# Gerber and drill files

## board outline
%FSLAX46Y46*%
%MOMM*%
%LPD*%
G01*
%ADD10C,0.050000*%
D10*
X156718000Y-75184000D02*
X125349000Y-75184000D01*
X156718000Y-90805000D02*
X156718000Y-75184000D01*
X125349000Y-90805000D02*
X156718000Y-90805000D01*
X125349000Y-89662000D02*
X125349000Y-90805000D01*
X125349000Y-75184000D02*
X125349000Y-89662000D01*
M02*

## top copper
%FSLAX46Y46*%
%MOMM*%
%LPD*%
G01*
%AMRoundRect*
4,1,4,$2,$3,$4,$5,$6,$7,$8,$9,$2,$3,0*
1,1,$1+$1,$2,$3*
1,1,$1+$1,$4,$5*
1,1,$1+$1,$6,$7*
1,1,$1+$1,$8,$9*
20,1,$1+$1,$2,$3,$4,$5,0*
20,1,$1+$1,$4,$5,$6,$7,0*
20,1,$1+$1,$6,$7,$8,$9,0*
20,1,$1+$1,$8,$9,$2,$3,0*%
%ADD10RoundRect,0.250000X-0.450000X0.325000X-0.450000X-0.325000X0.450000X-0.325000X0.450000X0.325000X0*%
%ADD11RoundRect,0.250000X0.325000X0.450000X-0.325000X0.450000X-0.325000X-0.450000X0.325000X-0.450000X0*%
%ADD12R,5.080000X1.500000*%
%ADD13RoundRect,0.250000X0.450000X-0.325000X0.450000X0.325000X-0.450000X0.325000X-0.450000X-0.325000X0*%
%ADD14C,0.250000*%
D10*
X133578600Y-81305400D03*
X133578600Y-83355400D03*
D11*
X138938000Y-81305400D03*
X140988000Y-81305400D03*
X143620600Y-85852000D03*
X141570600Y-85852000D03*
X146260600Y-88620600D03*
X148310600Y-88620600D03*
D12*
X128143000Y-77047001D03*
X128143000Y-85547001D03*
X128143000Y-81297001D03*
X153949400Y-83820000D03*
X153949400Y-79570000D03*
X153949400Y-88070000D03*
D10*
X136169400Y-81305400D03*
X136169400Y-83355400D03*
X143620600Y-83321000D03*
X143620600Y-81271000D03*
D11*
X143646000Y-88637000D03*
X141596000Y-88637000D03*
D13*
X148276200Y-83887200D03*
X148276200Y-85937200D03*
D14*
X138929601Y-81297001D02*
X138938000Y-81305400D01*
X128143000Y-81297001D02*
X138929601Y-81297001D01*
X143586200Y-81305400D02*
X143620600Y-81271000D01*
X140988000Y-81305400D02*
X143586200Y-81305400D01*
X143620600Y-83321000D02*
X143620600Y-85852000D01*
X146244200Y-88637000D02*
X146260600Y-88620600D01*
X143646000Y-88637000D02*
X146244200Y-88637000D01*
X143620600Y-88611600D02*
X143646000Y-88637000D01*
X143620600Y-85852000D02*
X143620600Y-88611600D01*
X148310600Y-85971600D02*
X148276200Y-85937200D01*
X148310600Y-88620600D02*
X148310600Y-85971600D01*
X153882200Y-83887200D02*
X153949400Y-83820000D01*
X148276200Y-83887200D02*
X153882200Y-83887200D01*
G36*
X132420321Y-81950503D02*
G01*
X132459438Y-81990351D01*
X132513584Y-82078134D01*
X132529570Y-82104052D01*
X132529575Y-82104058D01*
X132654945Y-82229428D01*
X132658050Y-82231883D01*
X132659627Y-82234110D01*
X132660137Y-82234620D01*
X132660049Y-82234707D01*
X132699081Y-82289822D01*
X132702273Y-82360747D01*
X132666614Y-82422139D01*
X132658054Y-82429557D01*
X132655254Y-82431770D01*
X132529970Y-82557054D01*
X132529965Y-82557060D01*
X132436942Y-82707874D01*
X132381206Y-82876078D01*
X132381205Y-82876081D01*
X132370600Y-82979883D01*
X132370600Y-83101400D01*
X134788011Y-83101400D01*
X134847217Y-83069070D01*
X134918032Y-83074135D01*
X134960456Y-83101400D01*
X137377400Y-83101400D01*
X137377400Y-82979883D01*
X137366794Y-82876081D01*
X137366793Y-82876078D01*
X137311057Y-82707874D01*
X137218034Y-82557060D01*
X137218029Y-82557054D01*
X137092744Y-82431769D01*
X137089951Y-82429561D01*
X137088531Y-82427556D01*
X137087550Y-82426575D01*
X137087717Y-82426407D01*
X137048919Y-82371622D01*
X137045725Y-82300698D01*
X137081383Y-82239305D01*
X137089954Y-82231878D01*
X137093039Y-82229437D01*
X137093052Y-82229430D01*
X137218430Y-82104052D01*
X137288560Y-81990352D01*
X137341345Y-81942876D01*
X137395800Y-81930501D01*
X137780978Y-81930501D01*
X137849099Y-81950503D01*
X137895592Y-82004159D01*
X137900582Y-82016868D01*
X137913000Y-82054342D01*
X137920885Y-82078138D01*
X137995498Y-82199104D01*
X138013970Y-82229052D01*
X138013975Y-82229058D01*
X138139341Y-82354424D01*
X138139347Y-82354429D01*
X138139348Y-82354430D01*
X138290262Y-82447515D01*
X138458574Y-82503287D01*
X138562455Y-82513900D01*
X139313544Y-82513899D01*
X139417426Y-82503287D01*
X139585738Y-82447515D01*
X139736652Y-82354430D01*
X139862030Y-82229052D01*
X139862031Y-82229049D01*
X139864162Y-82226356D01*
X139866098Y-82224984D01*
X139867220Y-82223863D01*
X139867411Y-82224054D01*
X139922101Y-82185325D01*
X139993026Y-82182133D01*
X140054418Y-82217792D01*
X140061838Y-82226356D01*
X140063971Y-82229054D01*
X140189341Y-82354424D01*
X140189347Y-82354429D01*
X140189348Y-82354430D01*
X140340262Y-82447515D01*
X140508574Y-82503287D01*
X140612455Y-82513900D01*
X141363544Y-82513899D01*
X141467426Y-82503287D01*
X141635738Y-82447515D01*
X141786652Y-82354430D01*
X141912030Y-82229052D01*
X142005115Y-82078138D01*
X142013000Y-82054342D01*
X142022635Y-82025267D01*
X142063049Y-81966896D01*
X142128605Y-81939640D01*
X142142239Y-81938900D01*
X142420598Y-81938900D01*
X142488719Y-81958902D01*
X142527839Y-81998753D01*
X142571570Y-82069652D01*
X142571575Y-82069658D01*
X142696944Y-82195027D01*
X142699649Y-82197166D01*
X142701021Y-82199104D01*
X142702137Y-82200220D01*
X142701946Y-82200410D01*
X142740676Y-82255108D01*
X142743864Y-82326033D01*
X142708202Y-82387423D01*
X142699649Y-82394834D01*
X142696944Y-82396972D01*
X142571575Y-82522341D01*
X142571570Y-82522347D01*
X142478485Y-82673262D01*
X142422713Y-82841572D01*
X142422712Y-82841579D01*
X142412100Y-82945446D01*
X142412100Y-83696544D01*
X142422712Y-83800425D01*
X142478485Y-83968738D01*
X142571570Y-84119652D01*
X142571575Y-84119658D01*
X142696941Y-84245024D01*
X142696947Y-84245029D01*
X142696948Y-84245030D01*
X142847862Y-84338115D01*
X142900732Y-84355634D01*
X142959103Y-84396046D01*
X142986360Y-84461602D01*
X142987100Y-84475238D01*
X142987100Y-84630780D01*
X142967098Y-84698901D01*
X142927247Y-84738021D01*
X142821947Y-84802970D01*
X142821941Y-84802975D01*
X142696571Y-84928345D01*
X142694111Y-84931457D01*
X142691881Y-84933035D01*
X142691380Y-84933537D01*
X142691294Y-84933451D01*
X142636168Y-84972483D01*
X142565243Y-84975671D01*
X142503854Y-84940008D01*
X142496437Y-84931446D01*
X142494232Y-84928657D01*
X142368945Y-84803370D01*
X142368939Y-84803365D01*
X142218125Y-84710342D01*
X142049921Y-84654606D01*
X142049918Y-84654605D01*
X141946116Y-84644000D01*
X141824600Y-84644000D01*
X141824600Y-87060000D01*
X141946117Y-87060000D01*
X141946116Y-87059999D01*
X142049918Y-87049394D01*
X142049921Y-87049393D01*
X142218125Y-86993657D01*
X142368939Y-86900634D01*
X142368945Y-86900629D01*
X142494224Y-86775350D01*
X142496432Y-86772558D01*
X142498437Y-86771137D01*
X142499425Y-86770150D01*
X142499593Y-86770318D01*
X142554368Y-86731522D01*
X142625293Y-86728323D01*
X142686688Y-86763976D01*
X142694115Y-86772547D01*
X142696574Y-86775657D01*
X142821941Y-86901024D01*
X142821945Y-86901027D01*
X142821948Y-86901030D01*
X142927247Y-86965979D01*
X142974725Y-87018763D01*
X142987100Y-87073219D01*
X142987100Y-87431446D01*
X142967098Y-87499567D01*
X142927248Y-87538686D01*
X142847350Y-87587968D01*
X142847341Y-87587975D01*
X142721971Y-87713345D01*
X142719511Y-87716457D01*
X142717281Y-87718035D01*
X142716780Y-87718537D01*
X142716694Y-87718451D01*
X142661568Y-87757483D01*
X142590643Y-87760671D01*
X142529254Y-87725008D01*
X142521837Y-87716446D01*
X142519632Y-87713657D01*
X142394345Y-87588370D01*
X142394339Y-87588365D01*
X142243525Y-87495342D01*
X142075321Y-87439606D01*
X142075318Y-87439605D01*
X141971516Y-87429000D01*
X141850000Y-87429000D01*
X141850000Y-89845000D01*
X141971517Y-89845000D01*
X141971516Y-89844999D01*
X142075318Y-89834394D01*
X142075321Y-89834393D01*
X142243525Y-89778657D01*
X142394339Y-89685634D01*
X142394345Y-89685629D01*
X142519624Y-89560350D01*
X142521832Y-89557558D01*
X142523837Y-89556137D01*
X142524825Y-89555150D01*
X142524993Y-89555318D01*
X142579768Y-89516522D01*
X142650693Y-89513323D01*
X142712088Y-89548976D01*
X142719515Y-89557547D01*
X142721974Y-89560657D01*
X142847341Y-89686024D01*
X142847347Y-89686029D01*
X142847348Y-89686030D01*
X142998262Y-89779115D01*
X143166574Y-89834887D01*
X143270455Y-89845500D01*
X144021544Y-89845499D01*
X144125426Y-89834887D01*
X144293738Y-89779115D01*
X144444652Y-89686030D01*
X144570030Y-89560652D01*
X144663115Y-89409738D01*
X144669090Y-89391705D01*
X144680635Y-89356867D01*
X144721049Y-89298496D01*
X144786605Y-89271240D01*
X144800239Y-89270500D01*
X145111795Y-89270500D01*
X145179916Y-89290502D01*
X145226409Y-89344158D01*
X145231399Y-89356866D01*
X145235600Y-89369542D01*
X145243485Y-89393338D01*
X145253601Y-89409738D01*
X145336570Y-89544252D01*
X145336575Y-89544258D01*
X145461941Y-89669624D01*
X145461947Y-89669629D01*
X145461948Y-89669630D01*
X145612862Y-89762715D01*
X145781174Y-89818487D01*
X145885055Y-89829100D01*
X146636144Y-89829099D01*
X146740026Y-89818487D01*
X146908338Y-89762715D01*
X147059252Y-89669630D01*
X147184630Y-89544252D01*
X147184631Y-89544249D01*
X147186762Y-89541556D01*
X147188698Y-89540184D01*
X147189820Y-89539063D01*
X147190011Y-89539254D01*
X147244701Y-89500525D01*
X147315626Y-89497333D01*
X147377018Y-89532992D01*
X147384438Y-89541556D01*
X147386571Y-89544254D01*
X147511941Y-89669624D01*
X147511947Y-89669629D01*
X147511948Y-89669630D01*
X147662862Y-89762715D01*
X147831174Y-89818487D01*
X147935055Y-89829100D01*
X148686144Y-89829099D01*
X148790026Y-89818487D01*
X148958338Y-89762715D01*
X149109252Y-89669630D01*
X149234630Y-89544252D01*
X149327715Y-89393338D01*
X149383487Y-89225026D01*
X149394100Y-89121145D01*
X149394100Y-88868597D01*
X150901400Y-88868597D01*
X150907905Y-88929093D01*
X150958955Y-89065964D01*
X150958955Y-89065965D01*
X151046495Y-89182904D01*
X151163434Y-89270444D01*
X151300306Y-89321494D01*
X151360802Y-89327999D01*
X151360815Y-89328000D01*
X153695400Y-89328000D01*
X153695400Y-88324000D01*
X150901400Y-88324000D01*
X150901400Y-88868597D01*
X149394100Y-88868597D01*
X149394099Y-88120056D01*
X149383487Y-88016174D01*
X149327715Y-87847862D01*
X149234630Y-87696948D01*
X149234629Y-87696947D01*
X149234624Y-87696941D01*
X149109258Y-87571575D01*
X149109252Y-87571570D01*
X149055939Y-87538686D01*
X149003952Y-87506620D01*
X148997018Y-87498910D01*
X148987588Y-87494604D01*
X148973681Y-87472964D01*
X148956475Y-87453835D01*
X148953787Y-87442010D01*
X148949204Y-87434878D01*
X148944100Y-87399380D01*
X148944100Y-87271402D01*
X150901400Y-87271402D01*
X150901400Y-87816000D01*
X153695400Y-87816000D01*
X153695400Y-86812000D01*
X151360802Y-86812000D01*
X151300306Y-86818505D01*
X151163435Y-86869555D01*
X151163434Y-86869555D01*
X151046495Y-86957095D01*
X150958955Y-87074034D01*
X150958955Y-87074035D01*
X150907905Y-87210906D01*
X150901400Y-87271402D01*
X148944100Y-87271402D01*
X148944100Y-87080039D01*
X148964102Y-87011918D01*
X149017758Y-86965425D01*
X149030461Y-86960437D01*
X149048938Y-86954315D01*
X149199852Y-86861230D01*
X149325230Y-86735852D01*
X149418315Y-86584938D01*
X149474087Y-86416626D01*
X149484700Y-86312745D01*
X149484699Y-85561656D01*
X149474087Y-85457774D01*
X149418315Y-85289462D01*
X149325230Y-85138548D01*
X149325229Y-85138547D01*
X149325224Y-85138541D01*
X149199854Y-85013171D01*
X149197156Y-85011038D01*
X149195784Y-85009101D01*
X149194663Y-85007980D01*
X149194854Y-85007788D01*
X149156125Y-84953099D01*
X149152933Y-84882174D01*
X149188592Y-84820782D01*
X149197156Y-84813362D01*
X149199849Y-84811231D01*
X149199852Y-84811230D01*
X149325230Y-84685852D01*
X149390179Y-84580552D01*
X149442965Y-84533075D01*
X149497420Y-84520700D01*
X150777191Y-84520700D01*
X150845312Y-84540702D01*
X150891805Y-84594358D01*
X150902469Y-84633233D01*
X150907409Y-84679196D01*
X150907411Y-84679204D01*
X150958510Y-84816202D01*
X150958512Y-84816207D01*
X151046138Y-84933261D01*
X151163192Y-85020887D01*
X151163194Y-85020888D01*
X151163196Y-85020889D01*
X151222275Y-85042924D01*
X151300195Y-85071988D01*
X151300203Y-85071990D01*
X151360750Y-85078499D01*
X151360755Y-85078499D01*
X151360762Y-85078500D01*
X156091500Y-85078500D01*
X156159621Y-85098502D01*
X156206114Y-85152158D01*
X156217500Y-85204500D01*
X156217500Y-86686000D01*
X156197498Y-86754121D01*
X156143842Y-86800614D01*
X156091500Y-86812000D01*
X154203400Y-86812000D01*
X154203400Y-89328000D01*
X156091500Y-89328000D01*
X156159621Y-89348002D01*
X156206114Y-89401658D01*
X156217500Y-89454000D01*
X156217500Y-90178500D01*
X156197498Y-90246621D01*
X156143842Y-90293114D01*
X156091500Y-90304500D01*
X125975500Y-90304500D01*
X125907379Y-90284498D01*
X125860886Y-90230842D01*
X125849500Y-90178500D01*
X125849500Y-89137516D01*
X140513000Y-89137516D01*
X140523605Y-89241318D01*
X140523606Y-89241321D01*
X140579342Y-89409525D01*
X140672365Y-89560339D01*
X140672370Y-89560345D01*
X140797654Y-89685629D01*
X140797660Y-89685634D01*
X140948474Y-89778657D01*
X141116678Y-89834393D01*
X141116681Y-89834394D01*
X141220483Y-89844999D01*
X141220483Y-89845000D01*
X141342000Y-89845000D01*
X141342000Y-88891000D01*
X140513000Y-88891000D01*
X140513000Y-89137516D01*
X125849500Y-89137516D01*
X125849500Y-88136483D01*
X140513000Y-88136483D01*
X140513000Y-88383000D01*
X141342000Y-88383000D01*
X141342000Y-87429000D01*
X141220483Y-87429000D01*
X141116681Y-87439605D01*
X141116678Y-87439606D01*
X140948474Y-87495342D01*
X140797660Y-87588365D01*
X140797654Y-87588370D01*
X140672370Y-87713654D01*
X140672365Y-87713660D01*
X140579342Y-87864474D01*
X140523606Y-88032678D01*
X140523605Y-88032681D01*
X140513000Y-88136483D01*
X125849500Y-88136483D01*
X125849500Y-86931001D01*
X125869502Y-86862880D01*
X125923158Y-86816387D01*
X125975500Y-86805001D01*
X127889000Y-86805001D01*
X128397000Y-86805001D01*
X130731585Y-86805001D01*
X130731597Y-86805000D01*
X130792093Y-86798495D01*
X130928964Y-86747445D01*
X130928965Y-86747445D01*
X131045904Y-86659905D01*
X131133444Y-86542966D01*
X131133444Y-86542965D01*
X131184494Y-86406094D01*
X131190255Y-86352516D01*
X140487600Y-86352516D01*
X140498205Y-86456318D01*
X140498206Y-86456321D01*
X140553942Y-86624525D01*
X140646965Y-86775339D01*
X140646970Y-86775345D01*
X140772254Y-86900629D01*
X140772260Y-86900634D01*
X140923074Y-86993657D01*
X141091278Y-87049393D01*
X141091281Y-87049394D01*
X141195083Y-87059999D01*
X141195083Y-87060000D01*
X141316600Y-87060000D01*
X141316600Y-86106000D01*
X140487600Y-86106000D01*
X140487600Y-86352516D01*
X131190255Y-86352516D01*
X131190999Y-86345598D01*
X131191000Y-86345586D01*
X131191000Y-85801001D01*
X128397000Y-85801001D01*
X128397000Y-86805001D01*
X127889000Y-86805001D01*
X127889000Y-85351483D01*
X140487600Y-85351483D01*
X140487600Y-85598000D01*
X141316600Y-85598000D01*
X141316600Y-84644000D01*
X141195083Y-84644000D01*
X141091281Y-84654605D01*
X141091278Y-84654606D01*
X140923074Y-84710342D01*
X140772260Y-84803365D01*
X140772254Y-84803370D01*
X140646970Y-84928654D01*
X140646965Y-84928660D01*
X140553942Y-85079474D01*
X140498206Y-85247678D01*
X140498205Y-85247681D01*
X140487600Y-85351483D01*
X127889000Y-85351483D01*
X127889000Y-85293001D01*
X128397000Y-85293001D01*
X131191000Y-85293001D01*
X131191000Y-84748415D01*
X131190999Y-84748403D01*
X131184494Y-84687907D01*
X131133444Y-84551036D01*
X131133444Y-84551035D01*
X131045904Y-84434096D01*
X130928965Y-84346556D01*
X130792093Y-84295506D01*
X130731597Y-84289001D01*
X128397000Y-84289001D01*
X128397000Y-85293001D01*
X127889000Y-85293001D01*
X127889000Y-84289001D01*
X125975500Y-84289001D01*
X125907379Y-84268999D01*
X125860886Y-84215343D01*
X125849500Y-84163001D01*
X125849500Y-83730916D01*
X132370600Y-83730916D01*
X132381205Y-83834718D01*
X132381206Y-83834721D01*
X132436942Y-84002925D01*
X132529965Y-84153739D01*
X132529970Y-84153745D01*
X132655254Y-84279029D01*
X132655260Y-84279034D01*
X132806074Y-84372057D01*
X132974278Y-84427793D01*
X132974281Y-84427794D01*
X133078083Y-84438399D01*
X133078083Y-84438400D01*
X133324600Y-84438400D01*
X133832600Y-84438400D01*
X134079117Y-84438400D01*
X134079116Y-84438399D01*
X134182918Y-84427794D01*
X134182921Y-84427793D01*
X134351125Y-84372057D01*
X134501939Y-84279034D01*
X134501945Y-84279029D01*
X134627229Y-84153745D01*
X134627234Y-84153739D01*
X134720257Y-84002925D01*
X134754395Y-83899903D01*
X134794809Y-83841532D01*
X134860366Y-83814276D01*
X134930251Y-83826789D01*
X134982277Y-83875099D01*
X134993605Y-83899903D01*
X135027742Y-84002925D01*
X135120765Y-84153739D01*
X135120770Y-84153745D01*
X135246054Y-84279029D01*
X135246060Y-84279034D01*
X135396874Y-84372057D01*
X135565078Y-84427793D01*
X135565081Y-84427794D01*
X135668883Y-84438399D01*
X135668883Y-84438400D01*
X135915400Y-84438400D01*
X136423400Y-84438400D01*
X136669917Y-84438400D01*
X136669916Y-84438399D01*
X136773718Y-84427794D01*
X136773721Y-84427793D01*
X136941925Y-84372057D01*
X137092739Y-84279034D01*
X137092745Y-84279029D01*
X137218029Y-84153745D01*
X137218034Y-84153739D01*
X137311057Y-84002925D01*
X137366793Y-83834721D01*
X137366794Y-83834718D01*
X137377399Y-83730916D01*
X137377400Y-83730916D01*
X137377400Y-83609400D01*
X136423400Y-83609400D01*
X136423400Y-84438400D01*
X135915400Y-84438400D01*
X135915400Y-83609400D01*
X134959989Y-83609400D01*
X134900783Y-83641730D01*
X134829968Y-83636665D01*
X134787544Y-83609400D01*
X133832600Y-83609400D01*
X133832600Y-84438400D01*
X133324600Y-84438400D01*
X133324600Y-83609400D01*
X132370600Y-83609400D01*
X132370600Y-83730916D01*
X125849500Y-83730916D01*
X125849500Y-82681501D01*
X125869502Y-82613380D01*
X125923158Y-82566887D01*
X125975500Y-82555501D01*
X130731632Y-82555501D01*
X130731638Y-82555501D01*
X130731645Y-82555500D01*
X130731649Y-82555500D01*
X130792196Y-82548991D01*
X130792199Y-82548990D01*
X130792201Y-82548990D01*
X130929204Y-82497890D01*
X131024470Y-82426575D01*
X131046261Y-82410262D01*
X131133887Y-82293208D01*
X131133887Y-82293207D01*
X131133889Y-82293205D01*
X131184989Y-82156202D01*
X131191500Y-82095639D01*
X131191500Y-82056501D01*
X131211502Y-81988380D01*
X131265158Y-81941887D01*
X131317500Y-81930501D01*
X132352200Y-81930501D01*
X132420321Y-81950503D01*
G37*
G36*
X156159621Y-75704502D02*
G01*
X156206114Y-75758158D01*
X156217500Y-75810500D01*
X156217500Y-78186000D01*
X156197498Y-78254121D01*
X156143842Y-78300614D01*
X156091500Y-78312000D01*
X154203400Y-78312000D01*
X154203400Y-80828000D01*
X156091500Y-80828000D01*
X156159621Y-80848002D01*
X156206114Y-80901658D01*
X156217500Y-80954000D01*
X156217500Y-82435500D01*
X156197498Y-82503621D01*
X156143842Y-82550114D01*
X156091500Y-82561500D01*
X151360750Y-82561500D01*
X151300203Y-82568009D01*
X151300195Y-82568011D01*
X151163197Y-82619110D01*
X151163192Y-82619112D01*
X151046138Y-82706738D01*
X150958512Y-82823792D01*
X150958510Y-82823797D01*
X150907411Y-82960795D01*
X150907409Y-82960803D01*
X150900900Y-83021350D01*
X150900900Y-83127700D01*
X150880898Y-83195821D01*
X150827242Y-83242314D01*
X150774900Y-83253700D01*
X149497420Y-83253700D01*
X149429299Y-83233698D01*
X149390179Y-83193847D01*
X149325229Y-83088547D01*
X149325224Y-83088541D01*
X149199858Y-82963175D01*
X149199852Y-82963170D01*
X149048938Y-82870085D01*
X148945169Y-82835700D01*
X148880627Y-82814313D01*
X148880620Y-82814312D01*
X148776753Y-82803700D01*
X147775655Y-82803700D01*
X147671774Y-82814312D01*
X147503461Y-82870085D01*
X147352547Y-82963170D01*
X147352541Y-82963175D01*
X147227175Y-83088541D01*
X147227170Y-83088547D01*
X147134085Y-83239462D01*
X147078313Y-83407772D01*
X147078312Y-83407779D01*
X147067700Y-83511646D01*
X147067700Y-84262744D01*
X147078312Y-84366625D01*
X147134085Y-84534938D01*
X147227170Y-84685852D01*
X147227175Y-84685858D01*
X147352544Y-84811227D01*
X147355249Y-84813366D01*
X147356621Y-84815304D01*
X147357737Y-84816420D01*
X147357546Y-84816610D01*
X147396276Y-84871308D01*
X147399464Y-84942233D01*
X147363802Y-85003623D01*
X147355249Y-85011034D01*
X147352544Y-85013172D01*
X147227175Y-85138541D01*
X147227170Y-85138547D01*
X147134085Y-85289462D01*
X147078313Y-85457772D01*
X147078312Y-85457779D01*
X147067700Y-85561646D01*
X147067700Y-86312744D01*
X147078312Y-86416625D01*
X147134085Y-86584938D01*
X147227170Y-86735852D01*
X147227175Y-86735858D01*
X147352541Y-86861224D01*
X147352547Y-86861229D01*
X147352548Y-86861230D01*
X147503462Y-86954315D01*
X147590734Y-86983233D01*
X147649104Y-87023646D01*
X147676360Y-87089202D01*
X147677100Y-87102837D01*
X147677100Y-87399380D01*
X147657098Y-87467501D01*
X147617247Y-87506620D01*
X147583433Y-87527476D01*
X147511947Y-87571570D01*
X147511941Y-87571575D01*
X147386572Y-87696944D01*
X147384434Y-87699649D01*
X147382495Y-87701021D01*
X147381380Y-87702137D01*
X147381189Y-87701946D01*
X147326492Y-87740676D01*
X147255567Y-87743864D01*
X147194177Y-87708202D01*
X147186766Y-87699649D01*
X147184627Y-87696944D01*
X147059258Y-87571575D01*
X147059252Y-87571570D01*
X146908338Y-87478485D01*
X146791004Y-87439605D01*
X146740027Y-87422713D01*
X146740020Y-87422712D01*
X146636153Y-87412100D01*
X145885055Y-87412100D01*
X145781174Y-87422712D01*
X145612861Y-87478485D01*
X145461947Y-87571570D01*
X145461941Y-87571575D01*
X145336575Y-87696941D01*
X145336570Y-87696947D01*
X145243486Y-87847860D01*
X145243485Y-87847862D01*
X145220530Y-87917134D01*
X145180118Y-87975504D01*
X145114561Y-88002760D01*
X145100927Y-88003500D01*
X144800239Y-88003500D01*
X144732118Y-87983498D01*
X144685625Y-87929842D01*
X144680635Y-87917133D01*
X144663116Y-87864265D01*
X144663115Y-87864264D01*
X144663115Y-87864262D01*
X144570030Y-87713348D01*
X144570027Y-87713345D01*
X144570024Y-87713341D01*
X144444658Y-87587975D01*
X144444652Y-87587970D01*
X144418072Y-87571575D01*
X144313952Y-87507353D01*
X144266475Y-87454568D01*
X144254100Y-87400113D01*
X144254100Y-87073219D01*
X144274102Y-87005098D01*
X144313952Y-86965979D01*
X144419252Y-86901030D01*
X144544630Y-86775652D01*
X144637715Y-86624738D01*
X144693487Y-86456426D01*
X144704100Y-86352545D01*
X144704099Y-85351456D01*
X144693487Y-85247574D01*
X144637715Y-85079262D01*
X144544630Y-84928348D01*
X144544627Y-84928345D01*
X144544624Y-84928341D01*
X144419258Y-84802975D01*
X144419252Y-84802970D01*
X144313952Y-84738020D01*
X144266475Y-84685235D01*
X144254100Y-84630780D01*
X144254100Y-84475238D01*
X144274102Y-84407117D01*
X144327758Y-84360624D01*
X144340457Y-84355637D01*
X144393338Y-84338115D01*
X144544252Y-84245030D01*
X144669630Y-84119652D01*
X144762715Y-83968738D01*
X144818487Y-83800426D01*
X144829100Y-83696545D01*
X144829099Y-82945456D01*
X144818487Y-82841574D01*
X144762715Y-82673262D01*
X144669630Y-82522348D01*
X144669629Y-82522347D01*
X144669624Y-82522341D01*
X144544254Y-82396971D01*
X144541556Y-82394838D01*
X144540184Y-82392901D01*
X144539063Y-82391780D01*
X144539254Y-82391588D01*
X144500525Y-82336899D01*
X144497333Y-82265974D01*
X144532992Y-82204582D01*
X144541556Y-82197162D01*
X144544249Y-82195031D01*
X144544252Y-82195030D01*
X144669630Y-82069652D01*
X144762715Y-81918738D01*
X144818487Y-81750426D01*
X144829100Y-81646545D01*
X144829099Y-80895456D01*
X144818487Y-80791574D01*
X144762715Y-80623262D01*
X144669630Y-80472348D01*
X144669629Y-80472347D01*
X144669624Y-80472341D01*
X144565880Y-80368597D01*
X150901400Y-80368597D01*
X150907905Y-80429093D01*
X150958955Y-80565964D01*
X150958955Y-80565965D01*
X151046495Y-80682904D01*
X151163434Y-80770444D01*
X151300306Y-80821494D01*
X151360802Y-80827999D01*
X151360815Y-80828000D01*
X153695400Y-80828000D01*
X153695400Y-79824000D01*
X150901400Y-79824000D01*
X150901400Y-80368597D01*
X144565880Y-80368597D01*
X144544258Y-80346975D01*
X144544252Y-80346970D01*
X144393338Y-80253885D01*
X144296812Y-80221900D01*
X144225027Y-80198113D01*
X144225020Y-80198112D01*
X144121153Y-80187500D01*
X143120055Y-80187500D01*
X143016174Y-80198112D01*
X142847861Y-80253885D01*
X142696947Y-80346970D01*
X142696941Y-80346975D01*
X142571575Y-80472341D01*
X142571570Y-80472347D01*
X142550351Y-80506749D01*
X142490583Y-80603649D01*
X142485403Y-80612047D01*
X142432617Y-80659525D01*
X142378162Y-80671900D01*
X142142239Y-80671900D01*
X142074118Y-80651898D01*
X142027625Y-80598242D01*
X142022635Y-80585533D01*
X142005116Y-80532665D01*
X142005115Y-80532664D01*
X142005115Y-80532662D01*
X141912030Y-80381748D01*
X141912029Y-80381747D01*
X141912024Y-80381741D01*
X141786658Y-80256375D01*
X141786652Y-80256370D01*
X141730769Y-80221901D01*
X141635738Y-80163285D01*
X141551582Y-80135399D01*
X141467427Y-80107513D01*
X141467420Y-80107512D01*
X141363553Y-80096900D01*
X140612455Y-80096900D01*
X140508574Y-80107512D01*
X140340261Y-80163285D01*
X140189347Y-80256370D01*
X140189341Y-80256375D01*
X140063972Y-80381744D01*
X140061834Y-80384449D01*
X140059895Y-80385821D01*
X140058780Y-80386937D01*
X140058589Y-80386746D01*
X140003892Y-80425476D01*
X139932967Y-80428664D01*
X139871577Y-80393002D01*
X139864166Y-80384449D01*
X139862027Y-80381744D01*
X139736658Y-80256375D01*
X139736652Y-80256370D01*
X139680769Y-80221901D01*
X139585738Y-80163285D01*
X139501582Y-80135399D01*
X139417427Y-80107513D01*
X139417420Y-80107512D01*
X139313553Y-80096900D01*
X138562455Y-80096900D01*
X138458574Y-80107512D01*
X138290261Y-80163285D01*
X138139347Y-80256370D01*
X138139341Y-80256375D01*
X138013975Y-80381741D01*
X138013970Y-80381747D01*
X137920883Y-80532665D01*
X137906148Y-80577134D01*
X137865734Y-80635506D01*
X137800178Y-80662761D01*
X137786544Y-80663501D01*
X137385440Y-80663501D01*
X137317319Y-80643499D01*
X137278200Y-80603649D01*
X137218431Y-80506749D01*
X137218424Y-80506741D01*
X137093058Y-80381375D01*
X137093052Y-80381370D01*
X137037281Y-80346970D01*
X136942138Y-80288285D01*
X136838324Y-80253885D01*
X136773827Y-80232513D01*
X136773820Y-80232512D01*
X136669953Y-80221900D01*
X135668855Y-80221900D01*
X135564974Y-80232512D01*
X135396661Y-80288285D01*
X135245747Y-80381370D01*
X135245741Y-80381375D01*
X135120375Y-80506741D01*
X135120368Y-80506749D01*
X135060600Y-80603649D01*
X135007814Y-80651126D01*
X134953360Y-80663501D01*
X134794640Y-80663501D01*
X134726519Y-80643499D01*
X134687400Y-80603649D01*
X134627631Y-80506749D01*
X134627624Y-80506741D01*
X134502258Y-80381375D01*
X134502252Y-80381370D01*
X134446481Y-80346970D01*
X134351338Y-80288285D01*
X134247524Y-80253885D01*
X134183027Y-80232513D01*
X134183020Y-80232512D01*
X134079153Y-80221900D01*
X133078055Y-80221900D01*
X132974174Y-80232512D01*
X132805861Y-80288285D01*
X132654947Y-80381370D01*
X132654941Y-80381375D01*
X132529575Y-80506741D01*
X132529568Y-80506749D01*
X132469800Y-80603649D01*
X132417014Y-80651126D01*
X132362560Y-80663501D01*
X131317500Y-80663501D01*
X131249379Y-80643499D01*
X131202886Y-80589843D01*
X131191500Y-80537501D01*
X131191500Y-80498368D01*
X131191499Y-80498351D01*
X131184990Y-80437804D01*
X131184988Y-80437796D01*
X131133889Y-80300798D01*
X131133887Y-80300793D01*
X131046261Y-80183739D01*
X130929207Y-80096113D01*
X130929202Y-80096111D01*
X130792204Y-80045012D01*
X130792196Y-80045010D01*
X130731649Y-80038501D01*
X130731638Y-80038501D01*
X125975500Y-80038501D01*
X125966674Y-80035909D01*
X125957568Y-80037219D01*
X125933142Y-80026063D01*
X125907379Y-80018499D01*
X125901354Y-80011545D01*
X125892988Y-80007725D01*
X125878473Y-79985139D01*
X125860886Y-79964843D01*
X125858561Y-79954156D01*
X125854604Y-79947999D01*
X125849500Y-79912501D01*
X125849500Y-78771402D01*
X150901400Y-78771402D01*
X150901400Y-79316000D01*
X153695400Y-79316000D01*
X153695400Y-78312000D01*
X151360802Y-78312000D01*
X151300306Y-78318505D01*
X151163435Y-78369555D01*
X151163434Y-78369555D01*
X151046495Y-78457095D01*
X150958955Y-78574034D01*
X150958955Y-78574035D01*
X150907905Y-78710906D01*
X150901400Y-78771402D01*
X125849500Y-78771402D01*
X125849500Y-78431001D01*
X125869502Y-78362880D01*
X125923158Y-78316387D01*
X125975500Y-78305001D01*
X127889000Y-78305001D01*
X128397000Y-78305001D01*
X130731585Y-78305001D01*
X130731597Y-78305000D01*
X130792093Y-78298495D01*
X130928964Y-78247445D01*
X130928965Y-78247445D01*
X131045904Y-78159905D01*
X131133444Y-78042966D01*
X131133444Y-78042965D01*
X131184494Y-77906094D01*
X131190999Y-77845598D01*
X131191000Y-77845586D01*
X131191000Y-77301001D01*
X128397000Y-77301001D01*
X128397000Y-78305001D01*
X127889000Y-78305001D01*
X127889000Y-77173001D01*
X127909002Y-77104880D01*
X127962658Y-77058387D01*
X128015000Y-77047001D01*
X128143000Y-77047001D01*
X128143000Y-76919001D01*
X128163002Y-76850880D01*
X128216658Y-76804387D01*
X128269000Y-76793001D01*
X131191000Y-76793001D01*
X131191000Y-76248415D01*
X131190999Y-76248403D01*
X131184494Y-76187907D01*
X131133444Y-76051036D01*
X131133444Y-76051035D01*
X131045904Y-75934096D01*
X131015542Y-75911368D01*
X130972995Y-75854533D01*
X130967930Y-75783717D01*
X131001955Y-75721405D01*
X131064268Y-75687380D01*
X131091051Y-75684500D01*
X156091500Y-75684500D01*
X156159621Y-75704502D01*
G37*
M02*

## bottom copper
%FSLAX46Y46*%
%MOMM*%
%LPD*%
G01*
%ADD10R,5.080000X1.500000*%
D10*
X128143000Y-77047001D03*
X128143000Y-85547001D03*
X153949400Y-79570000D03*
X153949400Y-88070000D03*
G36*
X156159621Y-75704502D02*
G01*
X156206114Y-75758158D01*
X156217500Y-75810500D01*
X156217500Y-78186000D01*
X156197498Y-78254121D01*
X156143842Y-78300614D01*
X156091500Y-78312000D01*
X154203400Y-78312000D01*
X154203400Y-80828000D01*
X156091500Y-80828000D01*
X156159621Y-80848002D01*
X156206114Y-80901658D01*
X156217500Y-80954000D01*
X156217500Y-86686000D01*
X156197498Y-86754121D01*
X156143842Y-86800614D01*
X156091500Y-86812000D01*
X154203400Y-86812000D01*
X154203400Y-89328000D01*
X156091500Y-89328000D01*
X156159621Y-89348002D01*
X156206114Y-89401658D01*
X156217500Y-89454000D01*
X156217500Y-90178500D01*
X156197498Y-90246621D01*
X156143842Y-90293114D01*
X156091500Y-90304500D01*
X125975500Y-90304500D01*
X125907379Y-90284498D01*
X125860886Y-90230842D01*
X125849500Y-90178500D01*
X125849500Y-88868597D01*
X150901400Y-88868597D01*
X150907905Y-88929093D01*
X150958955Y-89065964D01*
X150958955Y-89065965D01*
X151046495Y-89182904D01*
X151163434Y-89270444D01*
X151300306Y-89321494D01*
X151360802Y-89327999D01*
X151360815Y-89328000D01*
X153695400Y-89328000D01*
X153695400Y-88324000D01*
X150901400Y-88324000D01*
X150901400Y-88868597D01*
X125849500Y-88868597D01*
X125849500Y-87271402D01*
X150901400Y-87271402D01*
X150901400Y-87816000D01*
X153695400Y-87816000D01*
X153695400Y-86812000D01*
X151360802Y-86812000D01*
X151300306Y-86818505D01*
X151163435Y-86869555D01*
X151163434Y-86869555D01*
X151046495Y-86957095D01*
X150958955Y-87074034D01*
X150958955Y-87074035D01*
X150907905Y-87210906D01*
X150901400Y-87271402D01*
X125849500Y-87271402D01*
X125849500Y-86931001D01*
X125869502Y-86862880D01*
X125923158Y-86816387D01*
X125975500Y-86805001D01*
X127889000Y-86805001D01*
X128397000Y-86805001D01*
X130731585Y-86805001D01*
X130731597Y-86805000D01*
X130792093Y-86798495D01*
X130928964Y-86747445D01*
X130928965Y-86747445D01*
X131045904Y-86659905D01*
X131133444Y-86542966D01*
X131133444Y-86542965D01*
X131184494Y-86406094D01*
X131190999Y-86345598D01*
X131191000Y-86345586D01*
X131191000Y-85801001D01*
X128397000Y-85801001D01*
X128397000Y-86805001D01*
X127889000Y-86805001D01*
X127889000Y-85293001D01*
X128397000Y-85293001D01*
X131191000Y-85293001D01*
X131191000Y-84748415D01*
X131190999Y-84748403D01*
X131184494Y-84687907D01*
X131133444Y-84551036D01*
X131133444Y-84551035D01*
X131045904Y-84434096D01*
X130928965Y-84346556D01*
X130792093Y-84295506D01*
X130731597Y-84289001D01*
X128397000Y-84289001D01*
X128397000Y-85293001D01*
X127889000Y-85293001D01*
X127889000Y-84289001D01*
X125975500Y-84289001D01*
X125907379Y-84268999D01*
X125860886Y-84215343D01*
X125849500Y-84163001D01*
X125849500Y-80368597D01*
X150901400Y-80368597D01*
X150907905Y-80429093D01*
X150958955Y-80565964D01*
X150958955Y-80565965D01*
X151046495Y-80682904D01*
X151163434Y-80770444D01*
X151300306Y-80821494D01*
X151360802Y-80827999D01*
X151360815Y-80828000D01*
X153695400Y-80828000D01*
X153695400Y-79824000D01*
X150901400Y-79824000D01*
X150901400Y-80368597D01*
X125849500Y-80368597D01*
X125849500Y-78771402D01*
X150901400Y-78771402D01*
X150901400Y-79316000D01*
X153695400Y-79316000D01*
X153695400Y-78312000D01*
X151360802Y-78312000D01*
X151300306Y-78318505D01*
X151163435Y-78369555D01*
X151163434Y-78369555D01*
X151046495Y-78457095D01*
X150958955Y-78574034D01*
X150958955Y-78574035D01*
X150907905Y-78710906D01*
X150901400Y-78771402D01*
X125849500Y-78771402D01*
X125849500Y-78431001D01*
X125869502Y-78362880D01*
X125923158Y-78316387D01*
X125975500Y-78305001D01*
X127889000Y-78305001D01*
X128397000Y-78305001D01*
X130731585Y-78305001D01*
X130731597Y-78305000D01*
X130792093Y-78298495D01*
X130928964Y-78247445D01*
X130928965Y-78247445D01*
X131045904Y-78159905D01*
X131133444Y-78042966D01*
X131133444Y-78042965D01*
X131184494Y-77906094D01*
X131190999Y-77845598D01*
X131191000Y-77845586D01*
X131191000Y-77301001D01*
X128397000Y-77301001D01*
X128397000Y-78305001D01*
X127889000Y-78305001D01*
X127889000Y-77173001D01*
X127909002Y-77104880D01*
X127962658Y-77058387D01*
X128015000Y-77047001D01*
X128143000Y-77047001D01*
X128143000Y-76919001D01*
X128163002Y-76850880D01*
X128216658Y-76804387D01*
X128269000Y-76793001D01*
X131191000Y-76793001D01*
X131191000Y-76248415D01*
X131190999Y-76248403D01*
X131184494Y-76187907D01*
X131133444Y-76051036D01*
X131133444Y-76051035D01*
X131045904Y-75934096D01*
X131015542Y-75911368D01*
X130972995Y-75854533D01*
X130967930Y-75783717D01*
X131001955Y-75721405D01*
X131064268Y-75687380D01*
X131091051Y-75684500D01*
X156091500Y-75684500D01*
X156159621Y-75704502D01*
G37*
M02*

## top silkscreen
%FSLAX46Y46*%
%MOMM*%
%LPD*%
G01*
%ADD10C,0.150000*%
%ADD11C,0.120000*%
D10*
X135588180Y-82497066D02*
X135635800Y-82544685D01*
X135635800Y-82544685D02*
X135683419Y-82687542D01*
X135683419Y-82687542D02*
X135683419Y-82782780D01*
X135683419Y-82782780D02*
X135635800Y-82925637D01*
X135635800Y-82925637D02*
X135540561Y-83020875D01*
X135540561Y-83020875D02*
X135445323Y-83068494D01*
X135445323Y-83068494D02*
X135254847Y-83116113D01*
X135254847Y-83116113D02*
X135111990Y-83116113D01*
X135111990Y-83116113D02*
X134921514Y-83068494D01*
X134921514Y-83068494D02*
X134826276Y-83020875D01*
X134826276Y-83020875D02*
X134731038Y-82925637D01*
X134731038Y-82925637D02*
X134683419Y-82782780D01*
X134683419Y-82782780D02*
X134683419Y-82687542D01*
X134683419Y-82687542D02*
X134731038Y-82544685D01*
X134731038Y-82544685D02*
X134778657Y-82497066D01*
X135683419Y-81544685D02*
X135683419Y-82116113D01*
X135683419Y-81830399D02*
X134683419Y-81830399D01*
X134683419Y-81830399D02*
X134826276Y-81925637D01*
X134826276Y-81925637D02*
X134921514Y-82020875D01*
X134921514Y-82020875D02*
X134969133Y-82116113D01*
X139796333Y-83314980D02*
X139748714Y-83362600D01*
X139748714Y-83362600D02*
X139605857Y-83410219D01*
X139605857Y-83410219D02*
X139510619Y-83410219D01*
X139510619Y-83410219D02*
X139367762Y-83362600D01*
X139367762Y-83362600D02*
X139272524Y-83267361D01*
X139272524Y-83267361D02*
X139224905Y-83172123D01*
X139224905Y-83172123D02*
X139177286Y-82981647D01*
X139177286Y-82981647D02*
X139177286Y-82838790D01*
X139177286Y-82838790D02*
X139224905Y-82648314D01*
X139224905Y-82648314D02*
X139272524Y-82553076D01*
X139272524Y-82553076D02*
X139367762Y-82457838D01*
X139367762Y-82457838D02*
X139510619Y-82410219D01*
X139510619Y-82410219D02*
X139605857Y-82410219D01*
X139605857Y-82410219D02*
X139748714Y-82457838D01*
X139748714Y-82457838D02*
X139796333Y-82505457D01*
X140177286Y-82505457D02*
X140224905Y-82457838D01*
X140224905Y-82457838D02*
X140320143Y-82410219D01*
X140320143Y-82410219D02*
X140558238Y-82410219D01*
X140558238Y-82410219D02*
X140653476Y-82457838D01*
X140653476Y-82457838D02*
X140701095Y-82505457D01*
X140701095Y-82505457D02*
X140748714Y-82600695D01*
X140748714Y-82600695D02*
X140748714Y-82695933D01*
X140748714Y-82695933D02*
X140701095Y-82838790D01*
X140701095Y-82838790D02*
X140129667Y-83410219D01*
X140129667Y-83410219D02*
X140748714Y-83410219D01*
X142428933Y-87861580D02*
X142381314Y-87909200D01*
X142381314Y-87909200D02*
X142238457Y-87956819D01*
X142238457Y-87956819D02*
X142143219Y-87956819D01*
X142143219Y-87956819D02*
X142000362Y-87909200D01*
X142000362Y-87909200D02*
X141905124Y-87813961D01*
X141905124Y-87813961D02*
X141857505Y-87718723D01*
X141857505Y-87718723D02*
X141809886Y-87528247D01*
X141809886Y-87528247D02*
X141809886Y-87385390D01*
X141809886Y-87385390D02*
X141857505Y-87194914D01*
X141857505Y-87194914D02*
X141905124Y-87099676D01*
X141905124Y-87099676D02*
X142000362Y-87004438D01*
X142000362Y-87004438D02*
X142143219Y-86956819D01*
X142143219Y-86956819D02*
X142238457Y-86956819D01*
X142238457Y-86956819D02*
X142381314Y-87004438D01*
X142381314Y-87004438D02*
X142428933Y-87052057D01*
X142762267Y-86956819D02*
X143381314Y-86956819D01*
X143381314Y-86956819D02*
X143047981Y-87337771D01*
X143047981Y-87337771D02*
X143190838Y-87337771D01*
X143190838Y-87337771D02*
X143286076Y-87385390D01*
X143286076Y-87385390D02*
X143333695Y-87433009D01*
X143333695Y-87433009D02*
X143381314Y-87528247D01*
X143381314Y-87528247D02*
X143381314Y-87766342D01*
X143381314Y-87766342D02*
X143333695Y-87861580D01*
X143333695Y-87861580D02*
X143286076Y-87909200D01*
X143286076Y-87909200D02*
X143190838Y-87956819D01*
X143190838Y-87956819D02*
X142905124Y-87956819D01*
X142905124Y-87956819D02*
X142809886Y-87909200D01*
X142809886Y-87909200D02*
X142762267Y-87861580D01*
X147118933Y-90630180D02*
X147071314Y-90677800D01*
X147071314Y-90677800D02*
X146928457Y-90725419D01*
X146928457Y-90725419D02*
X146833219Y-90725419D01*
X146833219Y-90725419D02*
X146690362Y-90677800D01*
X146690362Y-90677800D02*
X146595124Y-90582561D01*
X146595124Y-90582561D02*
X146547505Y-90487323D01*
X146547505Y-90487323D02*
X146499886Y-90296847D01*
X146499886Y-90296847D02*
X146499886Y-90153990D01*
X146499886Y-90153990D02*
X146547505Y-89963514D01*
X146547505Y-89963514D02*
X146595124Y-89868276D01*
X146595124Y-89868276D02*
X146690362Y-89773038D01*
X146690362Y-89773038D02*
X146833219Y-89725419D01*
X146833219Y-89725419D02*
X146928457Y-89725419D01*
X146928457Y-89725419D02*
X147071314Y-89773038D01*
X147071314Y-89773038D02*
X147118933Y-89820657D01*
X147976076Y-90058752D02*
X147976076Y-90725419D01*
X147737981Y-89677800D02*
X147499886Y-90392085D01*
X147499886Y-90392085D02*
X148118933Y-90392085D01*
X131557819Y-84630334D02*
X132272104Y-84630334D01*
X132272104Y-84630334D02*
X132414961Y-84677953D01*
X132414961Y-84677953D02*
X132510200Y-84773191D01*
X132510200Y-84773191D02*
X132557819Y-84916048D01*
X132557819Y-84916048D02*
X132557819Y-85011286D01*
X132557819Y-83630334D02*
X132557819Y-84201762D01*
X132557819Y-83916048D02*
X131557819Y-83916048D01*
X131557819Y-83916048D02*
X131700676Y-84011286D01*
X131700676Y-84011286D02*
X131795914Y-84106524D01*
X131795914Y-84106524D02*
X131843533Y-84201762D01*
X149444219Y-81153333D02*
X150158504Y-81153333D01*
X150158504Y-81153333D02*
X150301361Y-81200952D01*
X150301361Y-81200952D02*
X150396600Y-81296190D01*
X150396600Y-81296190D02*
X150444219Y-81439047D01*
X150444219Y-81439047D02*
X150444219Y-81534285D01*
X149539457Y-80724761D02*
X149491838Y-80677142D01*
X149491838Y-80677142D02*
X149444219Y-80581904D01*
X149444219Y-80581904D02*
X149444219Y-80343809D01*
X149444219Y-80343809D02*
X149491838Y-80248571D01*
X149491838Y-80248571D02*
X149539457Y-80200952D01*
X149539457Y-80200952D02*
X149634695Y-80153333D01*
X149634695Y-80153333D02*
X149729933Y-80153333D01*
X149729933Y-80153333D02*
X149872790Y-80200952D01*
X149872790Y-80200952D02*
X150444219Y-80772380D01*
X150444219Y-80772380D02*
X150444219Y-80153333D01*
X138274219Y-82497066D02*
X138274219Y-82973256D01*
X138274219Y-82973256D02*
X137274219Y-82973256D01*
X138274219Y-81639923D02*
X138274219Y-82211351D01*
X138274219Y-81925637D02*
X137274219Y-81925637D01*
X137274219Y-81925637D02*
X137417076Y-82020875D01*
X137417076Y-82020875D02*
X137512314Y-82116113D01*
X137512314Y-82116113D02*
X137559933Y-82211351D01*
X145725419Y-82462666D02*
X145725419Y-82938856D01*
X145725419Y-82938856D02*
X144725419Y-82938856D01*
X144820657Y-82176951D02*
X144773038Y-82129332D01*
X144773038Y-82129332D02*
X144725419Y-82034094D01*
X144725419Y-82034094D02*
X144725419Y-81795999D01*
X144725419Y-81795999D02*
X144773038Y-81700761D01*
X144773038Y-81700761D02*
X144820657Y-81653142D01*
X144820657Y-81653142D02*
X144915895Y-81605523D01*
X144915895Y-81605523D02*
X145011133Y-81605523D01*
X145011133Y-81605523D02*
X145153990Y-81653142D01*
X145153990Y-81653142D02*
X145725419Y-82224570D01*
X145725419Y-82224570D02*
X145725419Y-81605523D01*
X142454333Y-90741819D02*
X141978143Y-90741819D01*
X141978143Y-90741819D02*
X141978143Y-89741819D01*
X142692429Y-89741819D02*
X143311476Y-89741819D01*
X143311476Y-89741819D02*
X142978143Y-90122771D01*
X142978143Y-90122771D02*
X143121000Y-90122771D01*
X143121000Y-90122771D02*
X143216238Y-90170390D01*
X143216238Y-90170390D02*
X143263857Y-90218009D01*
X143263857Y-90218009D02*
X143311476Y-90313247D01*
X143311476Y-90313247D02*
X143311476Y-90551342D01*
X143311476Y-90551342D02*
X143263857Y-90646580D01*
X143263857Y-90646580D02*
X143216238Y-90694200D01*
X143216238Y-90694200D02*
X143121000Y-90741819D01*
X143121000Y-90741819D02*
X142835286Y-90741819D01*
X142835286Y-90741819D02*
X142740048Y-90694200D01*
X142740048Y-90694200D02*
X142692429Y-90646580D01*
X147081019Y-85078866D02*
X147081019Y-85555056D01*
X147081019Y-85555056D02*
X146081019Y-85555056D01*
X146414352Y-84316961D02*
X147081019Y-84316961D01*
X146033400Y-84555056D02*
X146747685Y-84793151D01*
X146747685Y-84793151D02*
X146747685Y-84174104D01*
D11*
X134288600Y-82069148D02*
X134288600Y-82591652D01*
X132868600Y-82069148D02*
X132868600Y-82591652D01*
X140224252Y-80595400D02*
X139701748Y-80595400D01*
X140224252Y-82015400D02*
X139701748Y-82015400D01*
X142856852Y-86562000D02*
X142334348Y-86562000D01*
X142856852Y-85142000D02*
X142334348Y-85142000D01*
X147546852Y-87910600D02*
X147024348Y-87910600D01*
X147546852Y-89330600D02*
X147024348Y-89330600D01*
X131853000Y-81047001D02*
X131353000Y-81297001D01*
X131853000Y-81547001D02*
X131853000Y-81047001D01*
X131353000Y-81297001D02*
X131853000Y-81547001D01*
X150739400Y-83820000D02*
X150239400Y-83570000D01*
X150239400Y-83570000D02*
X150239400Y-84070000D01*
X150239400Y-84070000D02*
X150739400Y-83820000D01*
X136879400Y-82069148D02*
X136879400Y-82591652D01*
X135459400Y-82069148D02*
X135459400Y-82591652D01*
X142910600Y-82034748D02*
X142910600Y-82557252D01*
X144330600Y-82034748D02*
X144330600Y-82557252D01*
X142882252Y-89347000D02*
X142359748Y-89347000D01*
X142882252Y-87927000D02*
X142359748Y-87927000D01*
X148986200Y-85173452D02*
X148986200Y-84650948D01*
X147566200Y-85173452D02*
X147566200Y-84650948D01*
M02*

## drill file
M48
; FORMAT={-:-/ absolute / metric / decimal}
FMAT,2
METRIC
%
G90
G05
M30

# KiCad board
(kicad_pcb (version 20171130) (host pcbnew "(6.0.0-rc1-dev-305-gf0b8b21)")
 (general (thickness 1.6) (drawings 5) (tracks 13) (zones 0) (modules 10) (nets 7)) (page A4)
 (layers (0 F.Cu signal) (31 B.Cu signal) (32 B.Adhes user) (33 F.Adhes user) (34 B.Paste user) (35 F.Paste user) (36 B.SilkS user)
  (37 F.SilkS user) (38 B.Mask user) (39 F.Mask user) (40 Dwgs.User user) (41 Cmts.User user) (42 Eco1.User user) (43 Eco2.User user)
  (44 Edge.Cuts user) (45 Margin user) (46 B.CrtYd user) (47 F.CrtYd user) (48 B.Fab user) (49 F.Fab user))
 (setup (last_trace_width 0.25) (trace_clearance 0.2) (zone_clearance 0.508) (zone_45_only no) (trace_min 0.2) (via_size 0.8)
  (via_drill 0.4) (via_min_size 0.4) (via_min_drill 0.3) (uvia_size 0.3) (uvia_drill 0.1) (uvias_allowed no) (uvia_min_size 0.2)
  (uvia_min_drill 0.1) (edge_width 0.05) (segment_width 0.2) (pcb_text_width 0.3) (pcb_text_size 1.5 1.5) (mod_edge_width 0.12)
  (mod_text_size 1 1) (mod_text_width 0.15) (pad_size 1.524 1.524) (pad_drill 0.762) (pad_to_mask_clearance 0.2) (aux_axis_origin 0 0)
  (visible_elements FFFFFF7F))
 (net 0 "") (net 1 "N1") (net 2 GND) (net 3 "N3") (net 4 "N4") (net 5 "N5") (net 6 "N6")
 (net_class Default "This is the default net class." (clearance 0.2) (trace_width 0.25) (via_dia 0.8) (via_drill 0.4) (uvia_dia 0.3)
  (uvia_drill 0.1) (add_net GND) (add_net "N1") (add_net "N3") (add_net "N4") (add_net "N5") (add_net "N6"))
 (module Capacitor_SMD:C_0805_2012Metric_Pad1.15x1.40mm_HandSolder (layer F.Cu) (at 133.5786 82.3304 270)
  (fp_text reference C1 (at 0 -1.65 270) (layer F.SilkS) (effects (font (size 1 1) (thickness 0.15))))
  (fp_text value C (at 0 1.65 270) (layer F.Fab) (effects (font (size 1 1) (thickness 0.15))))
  (fp_line (start -0.261252 -0.71) (end 0.261252 -0.71) (layer F.SilkS) (width 0.12))
  (fp_line (start -0.261252 0.71) (end 0.261252 0.71) (layer F.SilkS) (width 0.12))
  (pad 1 smd roundrect (at -1.025 0 270) (size 1.15 1.4) (layers F.Cu F.Paste F.Mask) (roundrect_rratio 0.217391) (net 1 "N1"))
  (pad 2 smd roundrect (at 1.025 0 270) (size 1.15 1.4) (layers F.Cu F.Paste F.Mask) (roundrect_rratio 0.217391) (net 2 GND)))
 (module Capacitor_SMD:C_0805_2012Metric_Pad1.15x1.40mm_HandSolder (layer F.Cu) (at 139.963 81.3054 180)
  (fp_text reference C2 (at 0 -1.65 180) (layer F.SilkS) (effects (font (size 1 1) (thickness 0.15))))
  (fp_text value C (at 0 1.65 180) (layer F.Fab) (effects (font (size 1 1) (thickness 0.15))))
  (fp_line (start -0.261252 0.71) (end 0.261252 0.71) (layer F.SilkS) (width 0.12))
  (fp_line (start -0.261252 -0.71) (end 0.261252 -0.71) (layer F.SilkS) (width 0.12))
  (pad 2 smd roundrect (at 1.025 0 180) (size 1.15 1.4) (layers F.Cu F.Paste F.Mask) (roundrect_rratio 0.217391) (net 1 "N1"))
  (pad 1 smd roundrect (at -1.025 0 180) (size 1.15 1.4) (layers F.Cu F.Paste F.Mask) (roundrect_rratio 0.217391) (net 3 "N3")))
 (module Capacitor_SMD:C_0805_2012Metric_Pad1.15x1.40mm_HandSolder (layer F.Cu) (at 142.5956 85.852 180)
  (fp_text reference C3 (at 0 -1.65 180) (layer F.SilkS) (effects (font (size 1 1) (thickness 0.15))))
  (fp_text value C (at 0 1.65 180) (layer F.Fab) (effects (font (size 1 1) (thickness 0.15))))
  (fp_line (start -0.261252 -0.71) (end 0.261252 -0.71) (layer F.SilkS) (width 0.12))
  (fp_line (start -0.261252 0.71) (end 0.261252 0.71) (layer F.SilkS) (width 0.12))
  (pad 1 smd roundrect (at -1.025 0 180) (size 1.15 1.4) (layers F.Cu F.Paste F.Mask) (roundrect_rratio 0.217391) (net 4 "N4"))
  (pad 2 smd roundrect (at 1.025 0 180) (size 1.15 1.4) (layers F.Cu F.Paste F.Mask) (roundrect_rratio 0.217391) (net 2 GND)))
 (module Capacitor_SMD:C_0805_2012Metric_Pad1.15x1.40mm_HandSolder (layer F.Cu) (at 147.2856 88.6206 180)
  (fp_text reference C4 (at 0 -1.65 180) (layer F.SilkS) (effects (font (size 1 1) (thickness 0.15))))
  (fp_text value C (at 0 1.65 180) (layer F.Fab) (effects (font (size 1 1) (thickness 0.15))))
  (fp_line (start -0.261252 0.71) (end 0.261252 0.71) (layer F.SilkS) (width 0.12))
  (fp_line (start -0.261252 -0.71) (end 0.261252 -0.71) (layer F.SilkS) (width 0.12))
  (pad 2 smd roundrect (at 1.025 0 180) (size 1.15 1.4) (layers F.Cu F.Paste F.Mask) (roundrect_rratio 0.217391) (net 4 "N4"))
  (pad 1 smd roundrect (at -1.025 0 180) (size 1.15 1.4) (layers F.Cu F.Paste F.Mask) (roundrect_rratio 0.217391) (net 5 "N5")))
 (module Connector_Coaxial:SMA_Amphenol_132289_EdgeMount (layer F.Cu) (at 128.143 81.297001 180)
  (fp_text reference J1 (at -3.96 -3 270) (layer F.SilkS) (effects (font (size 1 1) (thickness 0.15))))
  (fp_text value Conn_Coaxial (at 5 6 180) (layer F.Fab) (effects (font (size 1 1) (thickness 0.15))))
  (fp_line (start -3.71 0.25) (end -3.21 0) (layer F.SilkS) (width 0.12))
  (fp_line (start -3.71 -0.25) (end -3.71 0.25) (layer F.SilkS) (width 0.12))
  (fp_line (start -3.21 0) (end -3.71 -0.25) (layer F.SilkS) (width 0.12))
  (pad 2 smd rect (at 0 4.25 270) (size 1.5 5.08) (layers B.Cu B.Paste B.Mask) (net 2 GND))
  (pad 2 smd rect (at 0 -4.25 270) (size 1.5 5.08) (layers B.Cu B.Paste B.Mask) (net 2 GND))
  (pad 2 smd rect (at 0 4.25 270) (size 1.5 5.08) (layers F.Cu F.Paste F.Mask) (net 2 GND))
  (pad 2 smd rect (at 0 -4.25 270) (size 1.5 5.08) (layers F.Cu F.Paste F.Mask) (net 2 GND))
  (pad 1 smd rect (at 0 0 270) (size 1.5 5.08) (layers F.Cu F.Paste F.Mask) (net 1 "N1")))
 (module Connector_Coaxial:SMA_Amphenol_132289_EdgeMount (layer F.Cu) (at 153.9494 83.82)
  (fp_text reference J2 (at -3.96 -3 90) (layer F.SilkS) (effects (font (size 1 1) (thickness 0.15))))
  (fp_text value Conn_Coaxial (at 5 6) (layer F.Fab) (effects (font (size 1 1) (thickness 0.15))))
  (fp_line (start -3.21 0) (end -3.71 -0.25) (layer F.SilkS) (width 0.12))
  (fp_line (start -3.71 -0.25) (end -3.71 0.25) (layer F.SilkS) (width 0.12))
  (fp_line (start -3.71 0.25) (end -3.21 0) (layer F.SilkS) (width 0.12))
  (pad 1 smd rect (at 0 0 90) (size 1.5 5.08) (layers F.Cu F.Paste F.Mask) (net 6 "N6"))
  (pad 2 smd rect (at 0 -4.25 90) (size 1.5 5.08) (layers F.Cu F.Paste F.Mask) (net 2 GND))
  (pad 2 smd rect (at 0 4.25 90) (size 1.5 5.08) (layers F.Cu F.Paste F.Mask) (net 2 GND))
  (pad 2 smd rect (at 0 -4.25 90) (size 1.5 5.08) (layers B.Cu B.Paste B.Mask) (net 2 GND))
  (pad 2 smd rect (at 0 4.25 90) (size 1.5 5.08) (layers B.Cu B.Paste B.Mask) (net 2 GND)))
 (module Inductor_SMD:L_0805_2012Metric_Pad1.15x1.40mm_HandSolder (layer F.Cu) (at 136.1694 82.3304 270)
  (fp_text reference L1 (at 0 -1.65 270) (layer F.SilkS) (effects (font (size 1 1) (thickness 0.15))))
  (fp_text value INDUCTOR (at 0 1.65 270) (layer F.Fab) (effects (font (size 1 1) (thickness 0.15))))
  (fp_line (start -0.261252 -0.71) (end 0.261252 -0.71) (layer F.SilkS) (width 0.12))
  (fp_line (start -0.261252 0.71) (end 0.261252 0.71) (layer F.SilkS) (width 0.12))
  (pad 1 smd roundrect (at -1.025 0 270) (size 1.15 1.4) (layers F.Cu F.Paste F.Mask) (roundrect_rratio 0.217391) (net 1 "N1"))
  (pad 2 smd roundrect (at 1.025 0 270) (size 1.15 1.4) (layers F.Cu F.Paste F.Mask) (roundrect_rratio 0.217391) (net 2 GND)))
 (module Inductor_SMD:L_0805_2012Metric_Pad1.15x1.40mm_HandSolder (layer F.Cu) (at 143.6206 82.296 270)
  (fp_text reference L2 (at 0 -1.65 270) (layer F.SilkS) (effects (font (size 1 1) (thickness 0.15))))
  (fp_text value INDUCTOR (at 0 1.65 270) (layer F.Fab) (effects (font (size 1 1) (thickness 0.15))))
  (fp_line (start -0.261252 0.71) (end 0.261252 0.71) (layer F.SilkS) (width 0.12))
  (fp_line (start -0.261252 -0.71) (end 0.261252 -0.71) (layer F.SilkS) (width 0.12))
  (pad 2 smd roundrect (at 1.025 0 270) (size 1.15 1.4) (layers F.Cu F.Paste F.Mask) (roundrect_rratio 0.217391) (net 4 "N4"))
  (pad 1 smd roundrect (at -1.025 0 270) (size 1.15 1.4) (layers F.Cu F.Paste F.Mask) (roundrect_rratio 0.217391) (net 3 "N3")))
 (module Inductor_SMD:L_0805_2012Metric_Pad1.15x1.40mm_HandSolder (layer F.Cu) (at 142.621 88.637 180)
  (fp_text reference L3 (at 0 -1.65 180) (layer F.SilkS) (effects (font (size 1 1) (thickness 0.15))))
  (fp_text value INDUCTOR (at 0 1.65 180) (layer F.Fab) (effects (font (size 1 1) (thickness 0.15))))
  (fp_line (start -0.261252 -0.71) (end 0.261252 -0.71) (layer F.SilkS) (width 0.12))
  (fp_line (start -0.261252 0.71) (end 0.261252 0.71) (layer F.SilkS) (width 0.12))
  (pad 1 smd roundrect (at -1.025 0 180) (size 1.15 1.4) (layers F.Cu F.Paste F.Mask) (roundrect_rratio 0.217391) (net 4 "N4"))
  (pad 2 smd roundrect (at 1.025 0 180) (size 1.15 1.4) (layers F.Cu F.Paste F.Mask) (roundrect_rratio 0.217391) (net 2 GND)))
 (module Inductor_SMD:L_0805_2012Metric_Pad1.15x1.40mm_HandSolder (layer F.Cu) (at 148.2762 84.9122 90)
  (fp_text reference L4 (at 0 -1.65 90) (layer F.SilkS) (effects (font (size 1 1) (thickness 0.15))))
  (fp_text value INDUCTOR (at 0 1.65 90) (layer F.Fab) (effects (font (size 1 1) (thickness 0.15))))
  (fp_line (start -0.261252 0.71) (end 0.261252 0.71) (layer F.SilkS) (width 0.12))
  (fp_line (start -0.261252 -0.71) (end 0.261252 -0.71) (layer F.SilkS) (width 0.12))
  (pad 2 smd roundrect (at 1.025 0 90) (size 1.15 1.4) (layers F.Cu F.Paste F.Mask) (roundrect_rratio 0.217391) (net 6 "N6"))
  (pad 1 smd roundrect (at -1.025 0 90) (size 1.15 1.4) (layers F.Cu F.Paste F.Mask) (roundrect_rratio 0.217391) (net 5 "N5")))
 (gr_line (start 156.718 75.184) (end 125.349 75.184) (layer Edge.Cuts) (width 0.05))
 (gr_line (start 156.718 90.805) (end 156.718 75.184) (layer Edge.Cuts) (width 0.05))
 (gr_line (start 125.349 90.805) (end 156.718 90.805) (layer Edge.Cuts) (width 0.05))
 (gr_line (start 125.349 89.662) (end 125.349 90.805) (layer Edge.Cuts) (width 0.05))
 (gr_line (start 125.349 75.184) (end 125.349 89.662) (layer Edge.Cuts) (width 0.05))
 (segment (start 138.929601 81.297001) (end 138.938 81.3054) (width 0.25) (layer F.Cu) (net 1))
 (segment (start 128.143 81.297001) (end 138.929601 81.297001) (width 0.25) (layer F.Cu) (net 1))
 (segment (start 143.5862 81.3054) (end 143.6206 81.271) (width 0.25) (layer F.Cu) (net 3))
 (segment (start 140.988 81.3054) (end 143.5862 81.3054) (width 0.25) (layer F.Cu) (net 3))
 (segment (start 143.6206 83.321) (end 143.6206 85.852) (width 0.25) (layer F.Cu) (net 4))
 (segment (start 146.2442 88.637) (end 146.2606 88.6206) (width 0.25) (layer F.Cu) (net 4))
 (segment (start 143.646 88.637) (end 146.2442 88.637) (width 0.25) (layer F.Cu) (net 4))
 (segment (start 143.6206 88.6116) (end 143.646 88.637) (width 0.25) (layer F.Cu) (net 4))
 (segment (start 143.6206 85.852) (end 143.6206 88.6116) (width 0.25) (layer F.Cu) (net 4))
 (segment (start 148.3106 85.9716) (end 148.2762 85.9372) (width 0.25) (layer F.Cu) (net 5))
 (segment (start 148.3106 88.6206) (end 148.3106 85.9716) (width 0.25) (layer F.Cu) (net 5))
 (segment (start 153.8822 83.8872) (end 153.9494 83.82) (width 0.25) (layer F.Cu) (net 6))
 (segment (start 148.2762 83.8872) (end 153.8822 83.8872) (width 0.25) (layer F.Cu) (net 6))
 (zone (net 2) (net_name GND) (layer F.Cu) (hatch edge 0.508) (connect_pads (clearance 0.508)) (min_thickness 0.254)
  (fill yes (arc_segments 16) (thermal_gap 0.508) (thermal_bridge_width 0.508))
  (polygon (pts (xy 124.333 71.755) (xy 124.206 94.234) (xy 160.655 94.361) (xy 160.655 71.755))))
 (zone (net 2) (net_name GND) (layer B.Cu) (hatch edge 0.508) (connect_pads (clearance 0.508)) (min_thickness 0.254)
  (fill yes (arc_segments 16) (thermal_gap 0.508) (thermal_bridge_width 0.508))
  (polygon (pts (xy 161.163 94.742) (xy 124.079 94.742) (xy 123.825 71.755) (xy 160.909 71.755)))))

